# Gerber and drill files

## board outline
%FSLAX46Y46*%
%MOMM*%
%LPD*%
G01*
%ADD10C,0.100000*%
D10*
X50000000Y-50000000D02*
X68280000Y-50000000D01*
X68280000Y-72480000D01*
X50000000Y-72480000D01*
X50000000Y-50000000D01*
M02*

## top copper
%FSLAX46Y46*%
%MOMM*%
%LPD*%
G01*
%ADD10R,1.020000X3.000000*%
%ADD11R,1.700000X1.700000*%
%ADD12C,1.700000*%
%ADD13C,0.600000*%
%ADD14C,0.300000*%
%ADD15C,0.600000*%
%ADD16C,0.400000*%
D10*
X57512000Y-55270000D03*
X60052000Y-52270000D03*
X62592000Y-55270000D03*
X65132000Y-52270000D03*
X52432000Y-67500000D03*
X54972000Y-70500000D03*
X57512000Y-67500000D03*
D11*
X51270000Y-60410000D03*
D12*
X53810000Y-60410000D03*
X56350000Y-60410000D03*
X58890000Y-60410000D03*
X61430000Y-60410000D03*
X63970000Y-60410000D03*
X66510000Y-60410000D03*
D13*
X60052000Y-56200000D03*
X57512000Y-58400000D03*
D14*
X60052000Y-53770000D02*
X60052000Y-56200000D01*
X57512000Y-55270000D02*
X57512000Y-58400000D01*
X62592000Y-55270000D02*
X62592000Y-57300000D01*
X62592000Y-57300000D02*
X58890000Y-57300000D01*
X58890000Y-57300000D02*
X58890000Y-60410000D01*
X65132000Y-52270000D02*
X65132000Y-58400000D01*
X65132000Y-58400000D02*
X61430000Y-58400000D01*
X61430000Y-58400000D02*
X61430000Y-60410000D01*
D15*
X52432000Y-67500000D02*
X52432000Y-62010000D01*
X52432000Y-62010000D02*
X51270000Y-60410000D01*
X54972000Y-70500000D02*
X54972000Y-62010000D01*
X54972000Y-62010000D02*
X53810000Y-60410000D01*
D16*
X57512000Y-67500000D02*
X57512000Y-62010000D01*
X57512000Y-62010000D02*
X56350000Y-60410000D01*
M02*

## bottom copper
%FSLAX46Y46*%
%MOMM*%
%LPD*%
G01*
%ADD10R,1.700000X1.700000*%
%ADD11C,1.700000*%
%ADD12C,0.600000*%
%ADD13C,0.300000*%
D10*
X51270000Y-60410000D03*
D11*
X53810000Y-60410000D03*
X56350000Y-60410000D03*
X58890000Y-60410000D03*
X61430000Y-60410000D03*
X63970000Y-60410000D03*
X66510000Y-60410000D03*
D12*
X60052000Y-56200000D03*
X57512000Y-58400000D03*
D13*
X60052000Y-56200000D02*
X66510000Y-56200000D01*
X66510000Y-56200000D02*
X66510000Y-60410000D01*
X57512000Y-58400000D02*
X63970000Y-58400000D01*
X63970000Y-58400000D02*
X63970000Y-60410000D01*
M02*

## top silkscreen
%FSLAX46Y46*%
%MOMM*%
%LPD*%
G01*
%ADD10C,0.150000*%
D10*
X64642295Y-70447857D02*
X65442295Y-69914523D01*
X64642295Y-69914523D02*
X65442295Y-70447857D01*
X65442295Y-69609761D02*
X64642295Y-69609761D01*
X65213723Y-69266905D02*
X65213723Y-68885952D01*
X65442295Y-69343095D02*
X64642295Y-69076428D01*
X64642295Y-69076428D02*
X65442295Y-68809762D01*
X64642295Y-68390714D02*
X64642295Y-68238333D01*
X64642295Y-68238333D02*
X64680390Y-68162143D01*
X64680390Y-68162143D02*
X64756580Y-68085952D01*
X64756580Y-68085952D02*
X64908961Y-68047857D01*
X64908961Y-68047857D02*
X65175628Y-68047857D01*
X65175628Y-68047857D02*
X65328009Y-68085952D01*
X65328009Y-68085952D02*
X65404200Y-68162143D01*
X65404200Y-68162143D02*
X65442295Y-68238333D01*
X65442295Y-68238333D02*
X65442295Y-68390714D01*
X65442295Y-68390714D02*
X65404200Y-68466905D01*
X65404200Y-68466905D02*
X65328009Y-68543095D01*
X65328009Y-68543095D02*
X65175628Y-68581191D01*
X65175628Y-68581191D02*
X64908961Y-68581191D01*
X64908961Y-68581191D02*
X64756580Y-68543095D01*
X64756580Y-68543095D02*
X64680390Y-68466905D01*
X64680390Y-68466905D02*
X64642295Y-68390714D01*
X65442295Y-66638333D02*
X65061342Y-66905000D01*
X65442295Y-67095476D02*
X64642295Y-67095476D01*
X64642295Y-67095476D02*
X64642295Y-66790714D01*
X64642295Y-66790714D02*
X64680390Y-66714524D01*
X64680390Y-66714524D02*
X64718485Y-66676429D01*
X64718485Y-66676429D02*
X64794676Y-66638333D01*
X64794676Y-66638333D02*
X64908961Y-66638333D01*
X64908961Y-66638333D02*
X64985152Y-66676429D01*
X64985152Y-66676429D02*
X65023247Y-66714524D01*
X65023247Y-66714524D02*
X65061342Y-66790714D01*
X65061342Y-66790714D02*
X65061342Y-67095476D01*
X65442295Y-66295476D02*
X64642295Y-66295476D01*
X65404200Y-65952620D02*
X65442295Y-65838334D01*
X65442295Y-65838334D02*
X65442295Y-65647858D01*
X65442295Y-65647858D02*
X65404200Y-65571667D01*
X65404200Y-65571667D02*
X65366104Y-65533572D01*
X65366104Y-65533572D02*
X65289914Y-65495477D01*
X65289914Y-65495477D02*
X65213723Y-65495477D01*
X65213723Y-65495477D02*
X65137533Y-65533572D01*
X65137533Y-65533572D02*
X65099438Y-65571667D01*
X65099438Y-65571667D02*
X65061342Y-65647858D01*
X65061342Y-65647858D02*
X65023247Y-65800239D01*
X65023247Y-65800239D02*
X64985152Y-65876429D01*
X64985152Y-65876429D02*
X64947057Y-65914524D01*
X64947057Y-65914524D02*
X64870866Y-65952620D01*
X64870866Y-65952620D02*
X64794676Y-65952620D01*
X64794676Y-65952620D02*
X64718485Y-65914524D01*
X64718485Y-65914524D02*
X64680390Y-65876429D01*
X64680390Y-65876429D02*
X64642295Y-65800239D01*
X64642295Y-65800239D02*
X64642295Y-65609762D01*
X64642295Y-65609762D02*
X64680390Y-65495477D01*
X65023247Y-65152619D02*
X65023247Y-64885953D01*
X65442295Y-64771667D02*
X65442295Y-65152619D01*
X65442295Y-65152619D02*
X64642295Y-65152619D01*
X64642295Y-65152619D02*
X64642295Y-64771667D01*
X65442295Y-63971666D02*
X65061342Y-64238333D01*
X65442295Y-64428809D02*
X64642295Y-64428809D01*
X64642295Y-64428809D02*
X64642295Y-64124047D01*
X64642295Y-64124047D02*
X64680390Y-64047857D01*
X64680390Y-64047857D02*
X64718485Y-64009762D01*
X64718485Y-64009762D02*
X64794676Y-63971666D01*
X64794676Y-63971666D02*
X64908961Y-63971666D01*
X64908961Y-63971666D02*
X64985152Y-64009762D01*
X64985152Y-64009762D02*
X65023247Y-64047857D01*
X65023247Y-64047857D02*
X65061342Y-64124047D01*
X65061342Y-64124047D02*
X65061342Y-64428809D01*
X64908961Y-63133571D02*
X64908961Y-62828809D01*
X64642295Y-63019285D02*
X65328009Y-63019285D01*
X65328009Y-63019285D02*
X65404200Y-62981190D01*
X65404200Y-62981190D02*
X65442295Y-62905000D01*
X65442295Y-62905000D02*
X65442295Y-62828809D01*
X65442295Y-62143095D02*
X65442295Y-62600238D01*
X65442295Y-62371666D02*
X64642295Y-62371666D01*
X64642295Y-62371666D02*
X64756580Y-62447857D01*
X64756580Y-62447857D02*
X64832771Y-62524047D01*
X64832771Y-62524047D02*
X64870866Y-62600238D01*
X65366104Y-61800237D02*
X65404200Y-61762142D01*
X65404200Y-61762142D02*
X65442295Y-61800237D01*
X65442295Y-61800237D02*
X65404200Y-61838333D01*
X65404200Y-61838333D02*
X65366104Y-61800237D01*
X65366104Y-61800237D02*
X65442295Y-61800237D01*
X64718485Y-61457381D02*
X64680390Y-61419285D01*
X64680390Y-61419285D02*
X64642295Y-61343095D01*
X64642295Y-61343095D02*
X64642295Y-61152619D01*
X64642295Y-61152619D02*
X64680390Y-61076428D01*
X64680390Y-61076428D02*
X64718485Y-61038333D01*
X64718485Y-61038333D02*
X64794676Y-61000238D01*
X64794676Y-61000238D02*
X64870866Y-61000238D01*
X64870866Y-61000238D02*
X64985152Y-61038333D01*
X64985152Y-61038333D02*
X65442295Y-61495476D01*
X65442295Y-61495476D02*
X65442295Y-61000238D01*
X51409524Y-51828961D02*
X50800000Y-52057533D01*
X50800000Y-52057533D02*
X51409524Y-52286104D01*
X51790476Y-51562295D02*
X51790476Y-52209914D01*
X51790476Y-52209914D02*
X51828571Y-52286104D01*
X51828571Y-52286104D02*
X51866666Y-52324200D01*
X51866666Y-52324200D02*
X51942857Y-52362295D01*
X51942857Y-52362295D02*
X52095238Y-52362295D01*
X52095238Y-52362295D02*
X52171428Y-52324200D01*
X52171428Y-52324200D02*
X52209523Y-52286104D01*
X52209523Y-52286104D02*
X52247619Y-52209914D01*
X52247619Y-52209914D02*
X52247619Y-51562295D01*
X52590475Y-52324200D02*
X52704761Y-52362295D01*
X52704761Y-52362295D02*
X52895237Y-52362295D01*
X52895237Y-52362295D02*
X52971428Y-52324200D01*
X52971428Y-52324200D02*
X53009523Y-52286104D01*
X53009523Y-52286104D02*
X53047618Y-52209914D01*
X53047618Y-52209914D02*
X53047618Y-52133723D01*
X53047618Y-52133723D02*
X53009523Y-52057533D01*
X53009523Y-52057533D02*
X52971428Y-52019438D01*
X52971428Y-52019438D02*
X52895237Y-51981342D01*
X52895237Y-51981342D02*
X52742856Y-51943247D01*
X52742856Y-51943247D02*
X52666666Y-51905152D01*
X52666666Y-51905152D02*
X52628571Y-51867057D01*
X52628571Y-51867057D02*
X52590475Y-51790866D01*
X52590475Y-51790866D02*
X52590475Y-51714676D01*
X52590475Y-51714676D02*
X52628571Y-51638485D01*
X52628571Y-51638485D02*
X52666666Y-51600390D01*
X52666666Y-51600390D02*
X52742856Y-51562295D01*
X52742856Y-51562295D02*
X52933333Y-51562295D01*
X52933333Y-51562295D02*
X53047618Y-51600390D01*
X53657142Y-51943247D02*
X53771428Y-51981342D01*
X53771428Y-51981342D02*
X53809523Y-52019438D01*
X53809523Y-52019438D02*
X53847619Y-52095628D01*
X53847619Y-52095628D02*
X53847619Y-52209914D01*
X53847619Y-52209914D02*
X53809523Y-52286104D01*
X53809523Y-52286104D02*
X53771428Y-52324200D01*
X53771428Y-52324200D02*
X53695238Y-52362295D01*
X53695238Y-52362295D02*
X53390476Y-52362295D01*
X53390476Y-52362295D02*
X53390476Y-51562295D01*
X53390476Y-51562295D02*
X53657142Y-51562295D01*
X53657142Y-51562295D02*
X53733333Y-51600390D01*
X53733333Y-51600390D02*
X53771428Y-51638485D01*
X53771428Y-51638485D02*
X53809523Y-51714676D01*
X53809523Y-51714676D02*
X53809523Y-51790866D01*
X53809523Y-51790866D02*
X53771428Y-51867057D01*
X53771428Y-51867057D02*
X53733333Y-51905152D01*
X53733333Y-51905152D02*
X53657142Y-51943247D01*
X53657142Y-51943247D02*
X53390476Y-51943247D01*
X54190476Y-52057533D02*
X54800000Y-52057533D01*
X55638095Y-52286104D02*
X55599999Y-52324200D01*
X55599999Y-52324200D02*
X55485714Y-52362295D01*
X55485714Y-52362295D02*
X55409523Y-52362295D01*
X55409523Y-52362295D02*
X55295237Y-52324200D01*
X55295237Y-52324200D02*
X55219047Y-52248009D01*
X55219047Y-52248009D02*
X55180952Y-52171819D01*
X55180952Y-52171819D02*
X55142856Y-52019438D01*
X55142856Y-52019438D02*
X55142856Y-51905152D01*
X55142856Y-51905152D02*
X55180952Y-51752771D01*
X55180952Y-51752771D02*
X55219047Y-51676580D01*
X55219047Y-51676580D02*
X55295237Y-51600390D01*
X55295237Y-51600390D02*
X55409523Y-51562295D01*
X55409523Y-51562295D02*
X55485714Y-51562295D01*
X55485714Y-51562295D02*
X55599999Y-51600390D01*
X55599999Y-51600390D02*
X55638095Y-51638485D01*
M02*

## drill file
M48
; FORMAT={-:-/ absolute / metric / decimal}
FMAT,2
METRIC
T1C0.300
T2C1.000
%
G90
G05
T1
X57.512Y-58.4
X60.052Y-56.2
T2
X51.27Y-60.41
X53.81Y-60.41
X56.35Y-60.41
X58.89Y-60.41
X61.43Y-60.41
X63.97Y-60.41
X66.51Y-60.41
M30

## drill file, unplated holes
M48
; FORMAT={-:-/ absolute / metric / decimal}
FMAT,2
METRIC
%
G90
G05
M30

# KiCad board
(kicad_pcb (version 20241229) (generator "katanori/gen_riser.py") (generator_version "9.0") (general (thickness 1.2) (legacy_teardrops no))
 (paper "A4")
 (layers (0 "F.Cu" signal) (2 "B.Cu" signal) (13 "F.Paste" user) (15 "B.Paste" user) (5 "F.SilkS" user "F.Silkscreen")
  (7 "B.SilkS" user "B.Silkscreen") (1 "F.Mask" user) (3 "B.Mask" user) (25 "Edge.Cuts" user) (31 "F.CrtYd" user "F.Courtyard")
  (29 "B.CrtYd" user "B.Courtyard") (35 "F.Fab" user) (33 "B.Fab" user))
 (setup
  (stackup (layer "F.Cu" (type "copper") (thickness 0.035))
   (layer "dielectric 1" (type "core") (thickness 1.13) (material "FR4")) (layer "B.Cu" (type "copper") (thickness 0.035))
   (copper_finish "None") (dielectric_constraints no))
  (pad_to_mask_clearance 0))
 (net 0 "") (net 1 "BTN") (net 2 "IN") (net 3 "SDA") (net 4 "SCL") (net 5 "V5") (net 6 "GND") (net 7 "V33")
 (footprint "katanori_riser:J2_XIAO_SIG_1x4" (layer "F.Cu") (at 50 50 0)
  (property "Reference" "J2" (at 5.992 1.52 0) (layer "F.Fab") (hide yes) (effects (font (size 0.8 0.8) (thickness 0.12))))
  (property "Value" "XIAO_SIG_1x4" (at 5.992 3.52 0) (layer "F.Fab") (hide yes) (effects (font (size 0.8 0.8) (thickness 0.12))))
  (pad "1" smd rect (at 7.512 5.27) (size 1.02 3) (layers "F.Cu" "F.Paste" "F.Mask") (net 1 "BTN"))
  (pad "2" smd rect (at 10.052 2.27) (size 1.02 3) (layers "F.Cu" "F.Paste" "F.Mask") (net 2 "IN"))
  (pad "3" smd rect (at 12.592 5.27) (size 1.02 3) (layers "F.Cu" "F.Paste" "F.Mask") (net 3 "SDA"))
  (pad "4" smd rect (at 15.132 2.27) (size 1.02 3) (layers "F.Cu" "F.Paste" "F.Mask") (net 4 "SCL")))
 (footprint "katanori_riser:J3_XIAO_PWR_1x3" (layer "F.Cu") (at 50 50 0)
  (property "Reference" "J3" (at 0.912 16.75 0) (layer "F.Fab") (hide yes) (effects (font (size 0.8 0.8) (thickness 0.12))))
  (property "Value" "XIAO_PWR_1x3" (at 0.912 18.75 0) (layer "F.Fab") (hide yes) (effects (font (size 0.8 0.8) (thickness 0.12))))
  (pad "1" smd rect (at 2.432 17.5) (size 1.02 3) (layers "F.Cu" "F.Paste" "F.Mask") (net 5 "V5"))
  (pad "2" smd rect (at 4.972 20.5) (size 1.02 3) (layers "F.Cu" "F.Paste" "F.Mask") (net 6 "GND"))
  (pad "3" smd rect (at 7.512 17.5) (size 1.02 3) (layers "F.Cu" "F.Paste" "F.Mask") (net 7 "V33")))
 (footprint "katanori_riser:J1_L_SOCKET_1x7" (layer "B.Cu") (at 50 50 0)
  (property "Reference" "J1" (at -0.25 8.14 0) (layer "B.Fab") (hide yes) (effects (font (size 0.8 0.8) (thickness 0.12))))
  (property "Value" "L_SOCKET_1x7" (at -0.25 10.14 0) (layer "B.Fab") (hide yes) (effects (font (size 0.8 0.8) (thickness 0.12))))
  (pad "1" thru_hole rect (at 1.27 10.41) (size 1.7 1.7) (drill 1) (layers "*.Cu" "*.Mask") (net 5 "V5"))
  (pad "2" thru_hole circle (at 3.81 10.41) (size 1.7 1.7) (drill 1) (layers "*.Cu" "*.Mask") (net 6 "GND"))
  (pad "3" thru_hole circle (at 6.35 10.41) (size 1.7 1.7) (drill 1) (layers "*.Cu" "*.Mask") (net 7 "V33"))
  (pad "4" thru_hole circle (at 8.89 10.41) (size 1.7 1.7) (drill 1) (layers "*.Cu" "*.Mask") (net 3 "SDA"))
  (pad "5" thru_hole circle (at 11.43 10.41) (size 1.7 1.7) (drill 1) (layers "*.Cu" "*.Mask") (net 4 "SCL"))
  (pad "6" thru_hole circle (at 13.97 10.41) (size 1.7 1.7) (drill 1) (layers "*.Cu" "*.Mask") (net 1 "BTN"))
  (pad "7" thru_hole circle (at 16.51 10.41) (size 1.7 1.7) (drill 1) (layers "*.Cu" "*.Mask") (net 2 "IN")))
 (segment (start 60.052 53.77) (end 60.052 56.2) (width 0.3) (layer "F.Cu") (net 2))
 (via (at 60.052 56.2) (size 0.6) (drill 0.3) (layers "F.Cu" "B.Cu") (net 2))
 (segment (start 60.052 56.2) (end 66.51 56.2) (width 0.3) (layer "B.Cu") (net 2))
 (segment (start 66.51 56.2) (end 66.51 60.41) (width 0.3) (layer "B.Cu") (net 2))
 (segment (start 57.512 55.27) (end 57.512 58.4) (width 0.3) (layer "F.Cu") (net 1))
 (via (at 57.512 58.4) (size 0.6) (drill 0.3) (layers "F.Cu" "B.Cu") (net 1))
 (segment (start 57.512 58.4) (end 63.97 58.4) (width 0.3) (layer "B.Cu") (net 1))
 (segment (start 63.97 58.4) (end 63.97 60.41) (width 0.3) (layer "B.Cu") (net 1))
 (segment (start 62.592 55.27) (end 62.592 57.3) (width 0.3) (layer "F.Cu") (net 3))
 (segment (start 62.592 57.3) (end 58.89 57.3) (width 0.3) (layer "F.Cu") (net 3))
 (segment (start 58.89 57.3) (end 58.89 60.41) (width 0.3) (layer "F.Cu") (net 3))
 (segment (start 65.132 52.27) (end 65.132 58.4) (width 0.3) (layer "F.Cu") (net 4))
 (segment (start 65.132 58.4) (end 61.43 58.4) (width 0.3) (layer "F.Cu") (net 4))
 (segment (start 61.43 58.4) (end 61.43 60.41) (width 0.3) (layer "F.Cu") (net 4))
 (segment (start 52.432 67.5) (end 52.432 62.01) (width 0.6) (layer "F.Cu") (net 5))
 (segment (start 52.432 62.01) (end 51.27 60.41) (width 0.6) (layer "F.Cu") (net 5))
 (segment (start 54.972 70.5) (end 54.972 62.01) (width 0.6) (layer "F.Cu") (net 6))
 (segment (start 54.972 62.01) (end 53.81 60.41) (width 0.6) (layer "F.Cu") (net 6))
 (segment (start 57.512 67.5) (end 57.512 62.01) (width 0.4) (layer "F.Cu") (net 7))
 (segment (start 57.512 62.01) (end 56.35 60.41) (width 0.4) (layer "F.Cu") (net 7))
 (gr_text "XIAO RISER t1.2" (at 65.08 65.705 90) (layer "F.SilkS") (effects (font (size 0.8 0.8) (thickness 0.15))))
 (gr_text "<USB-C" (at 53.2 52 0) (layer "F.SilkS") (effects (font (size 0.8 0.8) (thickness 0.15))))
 (gr_rect (start 50 50) (end 68.28 72.48) (stroke (width 0.1) (type default)) (fill no) (layer "Edge.Cuts")))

